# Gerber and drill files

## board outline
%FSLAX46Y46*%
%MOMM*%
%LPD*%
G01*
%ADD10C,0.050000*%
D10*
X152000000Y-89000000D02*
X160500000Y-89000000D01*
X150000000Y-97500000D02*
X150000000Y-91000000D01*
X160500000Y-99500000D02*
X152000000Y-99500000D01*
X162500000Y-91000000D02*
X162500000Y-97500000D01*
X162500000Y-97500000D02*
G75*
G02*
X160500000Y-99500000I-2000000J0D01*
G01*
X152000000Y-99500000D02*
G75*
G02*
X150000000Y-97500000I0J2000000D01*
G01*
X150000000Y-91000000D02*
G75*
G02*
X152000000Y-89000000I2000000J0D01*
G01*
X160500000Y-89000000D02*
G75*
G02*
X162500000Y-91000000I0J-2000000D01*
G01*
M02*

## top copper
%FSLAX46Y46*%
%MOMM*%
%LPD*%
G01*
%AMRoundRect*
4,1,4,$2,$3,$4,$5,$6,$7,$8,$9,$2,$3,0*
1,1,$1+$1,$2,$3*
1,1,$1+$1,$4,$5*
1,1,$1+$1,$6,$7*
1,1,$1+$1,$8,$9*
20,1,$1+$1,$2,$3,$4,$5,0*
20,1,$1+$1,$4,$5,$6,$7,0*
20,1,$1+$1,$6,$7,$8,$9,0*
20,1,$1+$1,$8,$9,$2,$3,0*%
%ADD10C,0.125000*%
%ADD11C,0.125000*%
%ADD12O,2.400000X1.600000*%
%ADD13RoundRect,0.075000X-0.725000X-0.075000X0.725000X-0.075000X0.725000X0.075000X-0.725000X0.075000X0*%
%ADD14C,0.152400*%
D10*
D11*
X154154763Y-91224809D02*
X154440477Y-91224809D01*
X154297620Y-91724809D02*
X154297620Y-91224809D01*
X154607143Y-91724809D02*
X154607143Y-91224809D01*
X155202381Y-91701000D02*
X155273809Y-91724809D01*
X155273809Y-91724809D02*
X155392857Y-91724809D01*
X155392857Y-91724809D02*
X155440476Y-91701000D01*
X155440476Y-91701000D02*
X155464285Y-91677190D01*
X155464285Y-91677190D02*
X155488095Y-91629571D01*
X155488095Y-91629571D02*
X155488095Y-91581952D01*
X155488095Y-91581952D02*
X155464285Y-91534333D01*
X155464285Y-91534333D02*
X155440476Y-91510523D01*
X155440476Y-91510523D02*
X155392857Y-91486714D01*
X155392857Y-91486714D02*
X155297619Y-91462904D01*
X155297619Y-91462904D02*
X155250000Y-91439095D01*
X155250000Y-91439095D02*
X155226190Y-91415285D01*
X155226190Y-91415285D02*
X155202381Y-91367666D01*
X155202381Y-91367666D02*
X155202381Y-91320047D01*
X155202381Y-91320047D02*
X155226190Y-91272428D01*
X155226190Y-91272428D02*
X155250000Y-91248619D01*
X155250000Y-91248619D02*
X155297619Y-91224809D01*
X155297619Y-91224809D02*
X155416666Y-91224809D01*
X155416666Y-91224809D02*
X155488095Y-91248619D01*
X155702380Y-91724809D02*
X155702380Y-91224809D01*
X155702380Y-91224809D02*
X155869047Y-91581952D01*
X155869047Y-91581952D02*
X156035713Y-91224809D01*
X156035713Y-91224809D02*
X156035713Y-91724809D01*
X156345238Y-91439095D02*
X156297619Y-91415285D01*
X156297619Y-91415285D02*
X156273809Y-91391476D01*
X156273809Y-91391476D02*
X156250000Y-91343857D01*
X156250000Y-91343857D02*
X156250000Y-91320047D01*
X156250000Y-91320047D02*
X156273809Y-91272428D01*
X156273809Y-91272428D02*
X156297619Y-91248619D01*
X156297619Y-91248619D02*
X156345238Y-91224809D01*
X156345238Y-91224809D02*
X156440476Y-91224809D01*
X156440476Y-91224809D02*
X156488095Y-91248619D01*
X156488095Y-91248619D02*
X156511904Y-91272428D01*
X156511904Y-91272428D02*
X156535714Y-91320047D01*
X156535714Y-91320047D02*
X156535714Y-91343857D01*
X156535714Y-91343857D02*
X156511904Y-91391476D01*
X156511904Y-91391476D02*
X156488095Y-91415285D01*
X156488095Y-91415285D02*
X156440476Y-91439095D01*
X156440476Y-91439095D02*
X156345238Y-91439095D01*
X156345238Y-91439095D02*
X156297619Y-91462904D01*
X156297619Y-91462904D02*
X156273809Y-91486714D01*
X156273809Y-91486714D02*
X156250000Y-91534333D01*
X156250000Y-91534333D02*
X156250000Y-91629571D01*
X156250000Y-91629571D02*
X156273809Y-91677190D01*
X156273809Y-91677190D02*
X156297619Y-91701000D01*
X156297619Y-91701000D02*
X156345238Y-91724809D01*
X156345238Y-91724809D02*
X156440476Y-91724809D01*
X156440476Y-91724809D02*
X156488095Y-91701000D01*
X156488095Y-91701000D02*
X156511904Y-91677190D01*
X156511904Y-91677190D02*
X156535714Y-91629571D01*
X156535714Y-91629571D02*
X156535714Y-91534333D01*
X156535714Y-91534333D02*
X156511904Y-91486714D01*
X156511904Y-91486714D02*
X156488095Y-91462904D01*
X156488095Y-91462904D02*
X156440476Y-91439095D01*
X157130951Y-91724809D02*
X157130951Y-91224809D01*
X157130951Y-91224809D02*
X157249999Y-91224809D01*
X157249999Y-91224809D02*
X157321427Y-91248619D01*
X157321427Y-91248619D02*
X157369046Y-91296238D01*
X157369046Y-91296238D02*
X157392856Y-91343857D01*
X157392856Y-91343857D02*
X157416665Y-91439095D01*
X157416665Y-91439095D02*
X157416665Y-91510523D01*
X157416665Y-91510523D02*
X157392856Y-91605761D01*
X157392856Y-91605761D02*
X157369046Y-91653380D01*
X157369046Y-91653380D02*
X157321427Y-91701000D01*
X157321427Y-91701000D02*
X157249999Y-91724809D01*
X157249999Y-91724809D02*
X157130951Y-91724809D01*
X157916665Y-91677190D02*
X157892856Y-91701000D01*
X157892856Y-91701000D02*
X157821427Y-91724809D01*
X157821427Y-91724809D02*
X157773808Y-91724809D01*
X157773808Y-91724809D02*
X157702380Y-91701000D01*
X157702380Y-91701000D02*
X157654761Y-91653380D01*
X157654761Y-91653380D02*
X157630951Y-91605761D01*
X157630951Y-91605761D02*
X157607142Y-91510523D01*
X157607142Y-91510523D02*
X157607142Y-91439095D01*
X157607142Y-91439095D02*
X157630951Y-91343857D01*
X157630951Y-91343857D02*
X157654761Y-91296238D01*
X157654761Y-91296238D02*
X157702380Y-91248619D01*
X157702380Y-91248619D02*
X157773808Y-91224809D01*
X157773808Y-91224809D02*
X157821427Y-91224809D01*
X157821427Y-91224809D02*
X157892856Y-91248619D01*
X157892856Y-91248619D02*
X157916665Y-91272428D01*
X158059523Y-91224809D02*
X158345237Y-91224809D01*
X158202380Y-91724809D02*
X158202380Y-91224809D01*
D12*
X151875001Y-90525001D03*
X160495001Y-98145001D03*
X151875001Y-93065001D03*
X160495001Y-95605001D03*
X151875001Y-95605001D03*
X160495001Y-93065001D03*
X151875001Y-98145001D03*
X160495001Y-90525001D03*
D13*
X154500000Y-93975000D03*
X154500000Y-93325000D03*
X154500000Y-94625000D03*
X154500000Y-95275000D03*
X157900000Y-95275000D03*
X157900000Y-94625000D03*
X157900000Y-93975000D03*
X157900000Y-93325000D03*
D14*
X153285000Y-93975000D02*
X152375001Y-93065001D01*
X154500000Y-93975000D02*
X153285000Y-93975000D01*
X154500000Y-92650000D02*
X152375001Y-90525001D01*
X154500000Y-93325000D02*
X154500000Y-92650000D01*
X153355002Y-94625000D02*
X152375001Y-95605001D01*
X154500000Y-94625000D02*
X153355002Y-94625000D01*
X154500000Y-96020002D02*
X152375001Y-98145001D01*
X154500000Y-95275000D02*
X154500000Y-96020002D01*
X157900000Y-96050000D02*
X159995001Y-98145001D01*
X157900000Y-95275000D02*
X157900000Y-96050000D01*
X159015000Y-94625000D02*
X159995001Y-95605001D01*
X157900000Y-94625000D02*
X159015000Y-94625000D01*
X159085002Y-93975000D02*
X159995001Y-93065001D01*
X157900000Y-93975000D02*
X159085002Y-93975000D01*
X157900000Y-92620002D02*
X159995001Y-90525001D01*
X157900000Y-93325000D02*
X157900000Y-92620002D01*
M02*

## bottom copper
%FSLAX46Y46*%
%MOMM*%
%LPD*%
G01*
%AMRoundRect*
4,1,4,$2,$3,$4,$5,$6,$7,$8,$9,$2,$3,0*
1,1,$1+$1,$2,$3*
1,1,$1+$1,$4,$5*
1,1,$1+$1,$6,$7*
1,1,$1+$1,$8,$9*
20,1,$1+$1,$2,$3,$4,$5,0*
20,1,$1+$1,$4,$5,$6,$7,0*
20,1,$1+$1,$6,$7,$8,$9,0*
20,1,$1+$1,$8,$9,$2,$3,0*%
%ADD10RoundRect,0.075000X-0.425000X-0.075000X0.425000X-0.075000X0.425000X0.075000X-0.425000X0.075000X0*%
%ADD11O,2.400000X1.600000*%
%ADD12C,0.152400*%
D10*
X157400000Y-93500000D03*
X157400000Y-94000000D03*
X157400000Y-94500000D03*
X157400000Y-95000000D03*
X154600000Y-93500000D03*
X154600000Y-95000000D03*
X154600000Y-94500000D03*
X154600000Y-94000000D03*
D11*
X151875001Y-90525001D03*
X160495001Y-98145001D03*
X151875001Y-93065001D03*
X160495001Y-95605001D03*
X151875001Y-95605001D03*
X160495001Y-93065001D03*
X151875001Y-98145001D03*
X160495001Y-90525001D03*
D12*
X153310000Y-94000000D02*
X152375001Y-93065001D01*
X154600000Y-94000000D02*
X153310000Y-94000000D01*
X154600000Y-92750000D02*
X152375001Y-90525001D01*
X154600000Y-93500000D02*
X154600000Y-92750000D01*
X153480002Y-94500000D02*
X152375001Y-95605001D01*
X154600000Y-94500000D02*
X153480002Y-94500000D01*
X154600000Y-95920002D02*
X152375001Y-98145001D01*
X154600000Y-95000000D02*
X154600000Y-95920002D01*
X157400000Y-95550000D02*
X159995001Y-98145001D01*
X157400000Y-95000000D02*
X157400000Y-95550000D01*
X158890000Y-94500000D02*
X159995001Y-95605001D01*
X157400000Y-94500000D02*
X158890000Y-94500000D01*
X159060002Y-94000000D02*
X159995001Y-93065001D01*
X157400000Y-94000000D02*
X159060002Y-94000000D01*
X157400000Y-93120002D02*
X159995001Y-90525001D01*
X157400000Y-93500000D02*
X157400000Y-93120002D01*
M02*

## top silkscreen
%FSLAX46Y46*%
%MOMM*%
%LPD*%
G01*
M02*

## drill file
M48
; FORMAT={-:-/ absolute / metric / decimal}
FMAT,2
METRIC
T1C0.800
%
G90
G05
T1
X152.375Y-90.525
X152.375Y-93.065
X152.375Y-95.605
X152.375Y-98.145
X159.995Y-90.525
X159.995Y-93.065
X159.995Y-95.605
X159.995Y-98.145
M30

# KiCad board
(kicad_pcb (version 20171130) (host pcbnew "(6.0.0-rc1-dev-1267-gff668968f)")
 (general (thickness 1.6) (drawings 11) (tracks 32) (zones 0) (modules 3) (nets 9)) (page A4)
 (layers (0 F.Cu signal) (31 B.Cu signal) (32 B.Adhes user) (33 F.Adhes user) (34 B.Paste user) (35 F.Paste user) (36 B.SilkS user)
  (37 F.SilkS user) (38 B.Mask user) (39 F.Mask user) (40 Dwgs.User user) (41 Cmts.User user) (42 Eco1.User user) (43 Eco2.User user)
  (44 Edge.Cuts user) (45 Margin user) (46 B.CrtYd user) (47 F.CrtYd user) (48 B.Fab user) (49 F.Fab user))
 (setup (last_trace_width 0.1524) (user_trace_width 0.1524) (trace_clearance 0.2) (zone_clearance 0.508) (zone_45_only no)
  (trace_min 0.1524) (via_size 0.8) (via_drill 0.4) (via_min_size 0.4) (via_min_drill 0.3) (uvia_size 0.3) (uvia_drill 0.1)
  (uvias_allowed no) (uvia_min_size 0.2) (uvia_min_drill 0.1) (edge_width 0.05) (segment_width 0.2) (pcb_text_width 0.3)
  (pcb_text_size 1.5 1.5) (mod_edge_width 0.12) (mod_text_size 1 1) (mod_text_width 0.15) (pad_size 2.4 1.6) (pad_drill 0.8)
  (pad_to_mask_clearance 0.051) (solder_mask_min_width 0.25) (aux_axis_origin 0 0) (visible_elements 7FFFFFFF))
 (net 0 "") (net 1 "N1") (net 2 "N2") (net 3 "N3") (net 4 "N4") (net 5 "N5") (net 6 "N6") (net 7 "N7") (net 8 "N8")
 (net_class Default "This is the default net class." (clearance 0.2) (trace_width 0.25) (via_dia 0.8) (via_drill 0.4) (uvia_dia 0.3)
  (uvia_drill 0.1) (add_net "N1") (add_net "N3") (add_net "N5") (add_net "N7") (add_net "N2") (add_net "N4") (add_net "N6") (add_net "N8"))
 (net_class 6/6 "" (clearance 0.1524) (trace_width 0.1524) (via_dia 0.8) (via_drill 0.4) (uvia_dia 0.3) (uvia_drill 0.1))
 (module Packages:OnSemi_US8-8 (layer B.Cu) (at 156 94.25)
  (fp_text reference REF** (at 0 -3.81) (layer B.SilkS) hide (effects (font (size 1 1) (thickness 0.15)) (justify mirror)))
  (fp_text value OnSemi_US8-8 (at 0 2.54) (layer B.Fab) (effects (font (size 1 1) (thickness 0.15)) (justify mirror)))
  (pad 5 smd roundrect (at 1.4 -0.75) (size 1 0.3) (layers B.Cu B.Paste B.Mask) (roundrect_rratio 0.25))
  (pad 6 smd roundrect (at 1.4 -0.25) (size 1 0.3) (layers B.Cu B.Paste B.Mask) (roundrect_rratio 0.25))
  (pad 7 smd roundrect (at 1.4 0.25) (size 1 0.3) (layers B.Cu B.Paste B.Mask) (roundrect_rratio 0.25))
  (pad 8 smd roundrect (at 1.4 0.75) (size 1 0.3) (layers B.Cu B.Paste B.Mask) (roundrect_rratio 0.25))
  (pad 4 smd roundrect (at -1.4 -0.75) (size 1 0.3) (layers B.Cu B.Paste B.Mask) (roundrect_rratio 0.25))
  (pad 1 smd roundrect (at -1.4 0.75) (size 1 0.3) (layers B.Cu B.Paste B.Mask) (roundrect_rratio 0.25))
  (pad 2 smd roundrect (at -1.4 0.25) (size 1 0.3) (layers B.Cu B.Paste B.Mask) (roundrect_rratio 0.25))
  (pad 3 smd roundrect (at -1.4 -0.25) (size 1 0.3) (layers B.Cu B.Paste B.Mask) (roundrect_rratio 0.25)))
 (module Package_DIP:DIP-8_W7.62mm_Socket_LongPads (layer F.Cu) (at 152.375001 90.525001)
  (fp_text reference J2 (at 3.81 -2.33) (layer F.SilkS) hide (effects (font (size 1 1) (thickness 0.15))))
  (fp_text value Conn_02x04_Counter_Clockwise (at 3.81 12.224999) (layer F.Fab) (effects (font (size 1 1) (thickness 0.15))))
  (pad 1 thru_hole oval (at 0 0) (size 2.4 1.6) (drill 0.8 (offset -0.5 0)) (layers *.Cu *.Mask) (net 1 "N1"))
  (pad 5 thru_hole oval (at 7.62 7.62) (size 2.4 1.6) (drill 0.8 (offset 0.5 0)) (layers *.Cu *.Mask) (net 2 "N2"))
  (pad 2 thru_hole oval (at 0 2.54) (size 2.4 1.6) (drill 0.8 (offset -0.5 0)) (layers *.Cu *.Mask) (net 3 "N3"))
  (pad 6 thru_hole oval (at 7.62 5.08) (size 2.4 1.6) (drill 0.8 (offset 0.5 0)) (layers *.Cu *.Mask) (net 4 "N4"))
  (pad 3 thru_hole oval (at 0 5.08) (size 2.4 1.6) (drill 0.8 (offset -0.5 0)) (layers *.Cu *.Mask) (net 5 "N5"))
  (pad 7 thru_hole oval (at 7.62 2.54) (size 2.4 1.6) (drill 0.8 (offset 0.5 0)) (layers *.Cu *.Mask) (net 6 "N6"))
  (pad 4 thru_hole oval (at 0 7.62) (size 2.4 1.6) (drill 0.8 (offset -0.5 0)) (layers *.Cu *.Mask) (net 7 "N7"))
  (pad 8 thru_hole oval (at 7.62 0) (size 2.4 1.6) (drill 0.8 (offset 0.5 0)) (layers *.Cu *.Mask) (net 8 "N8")))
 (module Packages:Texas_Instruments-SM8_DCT (layer F.Cu) (at 156.2 94.3)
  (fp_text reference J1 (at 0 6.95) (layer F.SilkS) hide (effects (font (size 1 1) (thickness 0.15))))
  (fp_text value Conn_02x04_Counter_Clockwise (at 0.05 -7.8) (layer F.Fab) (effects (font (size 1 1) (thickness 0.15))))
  (pad 2 smd roundrect (at -1.7 -0.325) (size 1.6 0.3) (layers F.Cu F.Paste F.Mask) (roundrect_rratio 0.25) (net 3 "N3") (clearance 0.07))
  (pad 1 smd roundrect (at -1.7 -0.975) (size 1.6 0.3) (layers F.Cu F.Paste F.Mask) (roundrect_rratio 0.25) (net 1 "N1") (clearance 0.07))
  (pad 3 smd roundrect (at -1.7 0.325) (size 1.6 0.3) (layers F.Cu F.Paste F.Mask) (roundrect_rratio 0.25) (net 5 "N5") (clearance 0.07))
  (pad 4 smd roundrect (at -1.7 0.975) (size 1.6 0.3) (layers F.Cu F.Paste F.Mask) (roundrect_rratio 0.25) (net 7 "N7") (clearance 0.07))
  (pad 5 smd roundrect (at 1.7 0.975) (size 1.6 0.3) (layers F.Cu F.Paste F.Mask) (roundrect_rratio 0.25) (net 2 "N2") (clearance 0.07))
  (pad 6 smd roundrect (at 1.7 0.325) (size 1.6 0.3) (layers F.Cu F.Paste F.Mask) (roundrect_rratio 0.25) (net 4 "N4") (clearance 0.07))
  (pad 7 smd roundrect (at 1.7 -0.325) (size 1.6 0.3) (layers F.Cu F.Paste F.Mask) (roundrect_rratio 0.25) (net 6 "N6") (clearance 0.07))
  (pad 8 smd roundrect (at 1.7 -0.975) (size 1.6 0.3) (layers F.Cu F.Paste F.Mask) (roundrect_rratio 0.25) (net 8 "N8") (clearance 0.07)))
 (gr_line (start 152 89) (end 160.5 89) (layer Edge.Cuts) (width 0.05))
 (gr_line (start 150 97.5) (end 150 91) (layer Edge.Cuts) (width 0.05))
 (gr_line (start 160.5 99.5) (end 152 99.5) (layer Edge.Cuts) (width 0.05))
 (gr_line (start 162.5 91) (end 162.5 97.5) (layer Edge.Cuts) (width 0.05))
 (gr_arc (start 160.5 97.5) (end 160.5 99.5) (angle -90) (layer Edge.Cuts) (width 0.05))
 (gr_arc (start 152 97.5) (end 150 97.5) (angle -90) (layer Edge.Cuts) (width 0.05))
 (gr_arc (start 152 91) (end 152 89) (angle -90) (layer Edge.Cuts) (width 0.05))
 (gr_arc (start 160.5 91) (end 162.5 91) (angle -90) (layer Edge.Cuts) (width 0.05))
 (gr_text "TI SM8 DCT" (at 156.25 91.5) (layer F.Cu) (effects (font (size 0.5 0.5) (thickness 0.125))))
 (segment (start 153.285 93.975) (end 152.375001 93.065001) (width 0.1524) (layer F.Cu) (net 3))
 (segment (start 154.5 93.975) (end 153.285 93.975) (width 0.1524) (layer F.Cu) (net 3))
 (segment (start 153.31 94) (end 152.375001 93.065001) (width 0.1524) (layer B.Cu) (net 3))
 (segment (start 154.6 94) (end 153.31 94) (width 0.1524) (layer B.Cu) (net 3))
 (segment (start 154.5 92.65) (end 152.375001 90.525001) (width 0.1524) (layer F.Cu) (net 1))
 (segment (start 154.5 93.325) (end 154.5 92.65) (width 0.1524) (layer F.Cu) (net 1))
 (segment (start 154.6 92.75) (end 152.375001 90.525001) (width 0.1524) (layer B.Cu) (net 1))
 (segment (start 154.6 93.5) (end 154.6 92.75) (width 0.1524) (layer B.Cu) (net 1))
 (segment (start 153.355002 94.625) (end 152.375001 95.605001) (width 0.1524) (layer F.Cu) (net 5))
 (segment (start 154.5 94.625) (end 153.355002 94.625) (width 0.1524) (layer F.Cu) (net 5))
 (segment (start 153.480002 94.5) (end 152.375001 95.605001) (width 0.1524) (layer B.Cu) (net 5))
 (segment (start 154.6 94.5) (end 153.480002 94.5) (width 0.1524) (layer B.Cu) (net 5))
 (segment (start 154.5 96.020002) (end 152.375001 98.145001) (width 0.1524) (layer F.Cu) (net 7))
 (segment (start 154.5 95.275) (end 154.5 96.020002) (width 0.1524) (layer F.Cu) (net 7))
 (segment (start 154.6 95.920002) (end 152.375001 98.145001) (width 0.1524) (layer B.Cu) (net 7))
 (segment (start 154.6 95) (end 154.6 95.920002) (width 0.1524) (layer B.Cu) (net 7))
 (segment (start 157.9 96.05) (end 159.995001 98.145001) (width 0.1524) (layer F.Cu) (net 2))
 (segment (start 157.9 95.275) (end 157.9 96.05) (width 0.1524) (layer F.Cu) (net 2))
 (segment (start 157.4 95.55) (end 159.995001 98.145001) (width 0.1524) (layer B.Cu) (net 2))
 (segment (start 157.4 95) (end 157.4 95.55) (width 0.1524) (layer B.Cu) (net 2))
 (segment (start 159.015 94.625) (end 159.995001 95.605001) (width 0.1524) (layer F.Cu) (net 4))
 (segment (start 157.9 94.625) (end 159.015 94.625) (width 0.1524) (layer F.Cu) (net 4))
 (segment (start 158.89 94.5) (end 159.995001 95.605001) (width 0.1524) (layer B.Cu) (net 4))
 (segment (start 157.4 94.5) (end 158.89 94.5) (width 0.1524) (layer B.Cu) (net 4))
 (segment (start 159.085002 93.975) (end 159.995001 93.065001) (width 0.1524) (layer F.Cu) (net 6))
 (segment (start 157.9 93.975) (end 159.085002 93.975) (width 0.1524) (layer F.Cu) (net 6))
 (segment (start 159.060002 94) (end 159.995001 93.065001) (width 0.1524) (layer B.Cu) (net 6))
 (segment (start 157.4 94) (end 159.060002 94) (width 0.1524) (layer B.Cu) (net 6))
 (segment (start 157.9 92.620002) (end 159.995001 90.525001) (width 0.1524) (layer F.Cu) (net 8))
 (segment (start 157.9 93.325) (end 157.9 92.620002) (width 0.1524) (layer F.Cu) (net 8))
 (segment (start 157.4 93.120002) (end 159.995001 90.525001) (width 0.1524) (layer B.Cu) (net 8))
 (segment (start 157.4 93.5) (end 157.4 93.120002) (width 0.1524) (layer B.Cu) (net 8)))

